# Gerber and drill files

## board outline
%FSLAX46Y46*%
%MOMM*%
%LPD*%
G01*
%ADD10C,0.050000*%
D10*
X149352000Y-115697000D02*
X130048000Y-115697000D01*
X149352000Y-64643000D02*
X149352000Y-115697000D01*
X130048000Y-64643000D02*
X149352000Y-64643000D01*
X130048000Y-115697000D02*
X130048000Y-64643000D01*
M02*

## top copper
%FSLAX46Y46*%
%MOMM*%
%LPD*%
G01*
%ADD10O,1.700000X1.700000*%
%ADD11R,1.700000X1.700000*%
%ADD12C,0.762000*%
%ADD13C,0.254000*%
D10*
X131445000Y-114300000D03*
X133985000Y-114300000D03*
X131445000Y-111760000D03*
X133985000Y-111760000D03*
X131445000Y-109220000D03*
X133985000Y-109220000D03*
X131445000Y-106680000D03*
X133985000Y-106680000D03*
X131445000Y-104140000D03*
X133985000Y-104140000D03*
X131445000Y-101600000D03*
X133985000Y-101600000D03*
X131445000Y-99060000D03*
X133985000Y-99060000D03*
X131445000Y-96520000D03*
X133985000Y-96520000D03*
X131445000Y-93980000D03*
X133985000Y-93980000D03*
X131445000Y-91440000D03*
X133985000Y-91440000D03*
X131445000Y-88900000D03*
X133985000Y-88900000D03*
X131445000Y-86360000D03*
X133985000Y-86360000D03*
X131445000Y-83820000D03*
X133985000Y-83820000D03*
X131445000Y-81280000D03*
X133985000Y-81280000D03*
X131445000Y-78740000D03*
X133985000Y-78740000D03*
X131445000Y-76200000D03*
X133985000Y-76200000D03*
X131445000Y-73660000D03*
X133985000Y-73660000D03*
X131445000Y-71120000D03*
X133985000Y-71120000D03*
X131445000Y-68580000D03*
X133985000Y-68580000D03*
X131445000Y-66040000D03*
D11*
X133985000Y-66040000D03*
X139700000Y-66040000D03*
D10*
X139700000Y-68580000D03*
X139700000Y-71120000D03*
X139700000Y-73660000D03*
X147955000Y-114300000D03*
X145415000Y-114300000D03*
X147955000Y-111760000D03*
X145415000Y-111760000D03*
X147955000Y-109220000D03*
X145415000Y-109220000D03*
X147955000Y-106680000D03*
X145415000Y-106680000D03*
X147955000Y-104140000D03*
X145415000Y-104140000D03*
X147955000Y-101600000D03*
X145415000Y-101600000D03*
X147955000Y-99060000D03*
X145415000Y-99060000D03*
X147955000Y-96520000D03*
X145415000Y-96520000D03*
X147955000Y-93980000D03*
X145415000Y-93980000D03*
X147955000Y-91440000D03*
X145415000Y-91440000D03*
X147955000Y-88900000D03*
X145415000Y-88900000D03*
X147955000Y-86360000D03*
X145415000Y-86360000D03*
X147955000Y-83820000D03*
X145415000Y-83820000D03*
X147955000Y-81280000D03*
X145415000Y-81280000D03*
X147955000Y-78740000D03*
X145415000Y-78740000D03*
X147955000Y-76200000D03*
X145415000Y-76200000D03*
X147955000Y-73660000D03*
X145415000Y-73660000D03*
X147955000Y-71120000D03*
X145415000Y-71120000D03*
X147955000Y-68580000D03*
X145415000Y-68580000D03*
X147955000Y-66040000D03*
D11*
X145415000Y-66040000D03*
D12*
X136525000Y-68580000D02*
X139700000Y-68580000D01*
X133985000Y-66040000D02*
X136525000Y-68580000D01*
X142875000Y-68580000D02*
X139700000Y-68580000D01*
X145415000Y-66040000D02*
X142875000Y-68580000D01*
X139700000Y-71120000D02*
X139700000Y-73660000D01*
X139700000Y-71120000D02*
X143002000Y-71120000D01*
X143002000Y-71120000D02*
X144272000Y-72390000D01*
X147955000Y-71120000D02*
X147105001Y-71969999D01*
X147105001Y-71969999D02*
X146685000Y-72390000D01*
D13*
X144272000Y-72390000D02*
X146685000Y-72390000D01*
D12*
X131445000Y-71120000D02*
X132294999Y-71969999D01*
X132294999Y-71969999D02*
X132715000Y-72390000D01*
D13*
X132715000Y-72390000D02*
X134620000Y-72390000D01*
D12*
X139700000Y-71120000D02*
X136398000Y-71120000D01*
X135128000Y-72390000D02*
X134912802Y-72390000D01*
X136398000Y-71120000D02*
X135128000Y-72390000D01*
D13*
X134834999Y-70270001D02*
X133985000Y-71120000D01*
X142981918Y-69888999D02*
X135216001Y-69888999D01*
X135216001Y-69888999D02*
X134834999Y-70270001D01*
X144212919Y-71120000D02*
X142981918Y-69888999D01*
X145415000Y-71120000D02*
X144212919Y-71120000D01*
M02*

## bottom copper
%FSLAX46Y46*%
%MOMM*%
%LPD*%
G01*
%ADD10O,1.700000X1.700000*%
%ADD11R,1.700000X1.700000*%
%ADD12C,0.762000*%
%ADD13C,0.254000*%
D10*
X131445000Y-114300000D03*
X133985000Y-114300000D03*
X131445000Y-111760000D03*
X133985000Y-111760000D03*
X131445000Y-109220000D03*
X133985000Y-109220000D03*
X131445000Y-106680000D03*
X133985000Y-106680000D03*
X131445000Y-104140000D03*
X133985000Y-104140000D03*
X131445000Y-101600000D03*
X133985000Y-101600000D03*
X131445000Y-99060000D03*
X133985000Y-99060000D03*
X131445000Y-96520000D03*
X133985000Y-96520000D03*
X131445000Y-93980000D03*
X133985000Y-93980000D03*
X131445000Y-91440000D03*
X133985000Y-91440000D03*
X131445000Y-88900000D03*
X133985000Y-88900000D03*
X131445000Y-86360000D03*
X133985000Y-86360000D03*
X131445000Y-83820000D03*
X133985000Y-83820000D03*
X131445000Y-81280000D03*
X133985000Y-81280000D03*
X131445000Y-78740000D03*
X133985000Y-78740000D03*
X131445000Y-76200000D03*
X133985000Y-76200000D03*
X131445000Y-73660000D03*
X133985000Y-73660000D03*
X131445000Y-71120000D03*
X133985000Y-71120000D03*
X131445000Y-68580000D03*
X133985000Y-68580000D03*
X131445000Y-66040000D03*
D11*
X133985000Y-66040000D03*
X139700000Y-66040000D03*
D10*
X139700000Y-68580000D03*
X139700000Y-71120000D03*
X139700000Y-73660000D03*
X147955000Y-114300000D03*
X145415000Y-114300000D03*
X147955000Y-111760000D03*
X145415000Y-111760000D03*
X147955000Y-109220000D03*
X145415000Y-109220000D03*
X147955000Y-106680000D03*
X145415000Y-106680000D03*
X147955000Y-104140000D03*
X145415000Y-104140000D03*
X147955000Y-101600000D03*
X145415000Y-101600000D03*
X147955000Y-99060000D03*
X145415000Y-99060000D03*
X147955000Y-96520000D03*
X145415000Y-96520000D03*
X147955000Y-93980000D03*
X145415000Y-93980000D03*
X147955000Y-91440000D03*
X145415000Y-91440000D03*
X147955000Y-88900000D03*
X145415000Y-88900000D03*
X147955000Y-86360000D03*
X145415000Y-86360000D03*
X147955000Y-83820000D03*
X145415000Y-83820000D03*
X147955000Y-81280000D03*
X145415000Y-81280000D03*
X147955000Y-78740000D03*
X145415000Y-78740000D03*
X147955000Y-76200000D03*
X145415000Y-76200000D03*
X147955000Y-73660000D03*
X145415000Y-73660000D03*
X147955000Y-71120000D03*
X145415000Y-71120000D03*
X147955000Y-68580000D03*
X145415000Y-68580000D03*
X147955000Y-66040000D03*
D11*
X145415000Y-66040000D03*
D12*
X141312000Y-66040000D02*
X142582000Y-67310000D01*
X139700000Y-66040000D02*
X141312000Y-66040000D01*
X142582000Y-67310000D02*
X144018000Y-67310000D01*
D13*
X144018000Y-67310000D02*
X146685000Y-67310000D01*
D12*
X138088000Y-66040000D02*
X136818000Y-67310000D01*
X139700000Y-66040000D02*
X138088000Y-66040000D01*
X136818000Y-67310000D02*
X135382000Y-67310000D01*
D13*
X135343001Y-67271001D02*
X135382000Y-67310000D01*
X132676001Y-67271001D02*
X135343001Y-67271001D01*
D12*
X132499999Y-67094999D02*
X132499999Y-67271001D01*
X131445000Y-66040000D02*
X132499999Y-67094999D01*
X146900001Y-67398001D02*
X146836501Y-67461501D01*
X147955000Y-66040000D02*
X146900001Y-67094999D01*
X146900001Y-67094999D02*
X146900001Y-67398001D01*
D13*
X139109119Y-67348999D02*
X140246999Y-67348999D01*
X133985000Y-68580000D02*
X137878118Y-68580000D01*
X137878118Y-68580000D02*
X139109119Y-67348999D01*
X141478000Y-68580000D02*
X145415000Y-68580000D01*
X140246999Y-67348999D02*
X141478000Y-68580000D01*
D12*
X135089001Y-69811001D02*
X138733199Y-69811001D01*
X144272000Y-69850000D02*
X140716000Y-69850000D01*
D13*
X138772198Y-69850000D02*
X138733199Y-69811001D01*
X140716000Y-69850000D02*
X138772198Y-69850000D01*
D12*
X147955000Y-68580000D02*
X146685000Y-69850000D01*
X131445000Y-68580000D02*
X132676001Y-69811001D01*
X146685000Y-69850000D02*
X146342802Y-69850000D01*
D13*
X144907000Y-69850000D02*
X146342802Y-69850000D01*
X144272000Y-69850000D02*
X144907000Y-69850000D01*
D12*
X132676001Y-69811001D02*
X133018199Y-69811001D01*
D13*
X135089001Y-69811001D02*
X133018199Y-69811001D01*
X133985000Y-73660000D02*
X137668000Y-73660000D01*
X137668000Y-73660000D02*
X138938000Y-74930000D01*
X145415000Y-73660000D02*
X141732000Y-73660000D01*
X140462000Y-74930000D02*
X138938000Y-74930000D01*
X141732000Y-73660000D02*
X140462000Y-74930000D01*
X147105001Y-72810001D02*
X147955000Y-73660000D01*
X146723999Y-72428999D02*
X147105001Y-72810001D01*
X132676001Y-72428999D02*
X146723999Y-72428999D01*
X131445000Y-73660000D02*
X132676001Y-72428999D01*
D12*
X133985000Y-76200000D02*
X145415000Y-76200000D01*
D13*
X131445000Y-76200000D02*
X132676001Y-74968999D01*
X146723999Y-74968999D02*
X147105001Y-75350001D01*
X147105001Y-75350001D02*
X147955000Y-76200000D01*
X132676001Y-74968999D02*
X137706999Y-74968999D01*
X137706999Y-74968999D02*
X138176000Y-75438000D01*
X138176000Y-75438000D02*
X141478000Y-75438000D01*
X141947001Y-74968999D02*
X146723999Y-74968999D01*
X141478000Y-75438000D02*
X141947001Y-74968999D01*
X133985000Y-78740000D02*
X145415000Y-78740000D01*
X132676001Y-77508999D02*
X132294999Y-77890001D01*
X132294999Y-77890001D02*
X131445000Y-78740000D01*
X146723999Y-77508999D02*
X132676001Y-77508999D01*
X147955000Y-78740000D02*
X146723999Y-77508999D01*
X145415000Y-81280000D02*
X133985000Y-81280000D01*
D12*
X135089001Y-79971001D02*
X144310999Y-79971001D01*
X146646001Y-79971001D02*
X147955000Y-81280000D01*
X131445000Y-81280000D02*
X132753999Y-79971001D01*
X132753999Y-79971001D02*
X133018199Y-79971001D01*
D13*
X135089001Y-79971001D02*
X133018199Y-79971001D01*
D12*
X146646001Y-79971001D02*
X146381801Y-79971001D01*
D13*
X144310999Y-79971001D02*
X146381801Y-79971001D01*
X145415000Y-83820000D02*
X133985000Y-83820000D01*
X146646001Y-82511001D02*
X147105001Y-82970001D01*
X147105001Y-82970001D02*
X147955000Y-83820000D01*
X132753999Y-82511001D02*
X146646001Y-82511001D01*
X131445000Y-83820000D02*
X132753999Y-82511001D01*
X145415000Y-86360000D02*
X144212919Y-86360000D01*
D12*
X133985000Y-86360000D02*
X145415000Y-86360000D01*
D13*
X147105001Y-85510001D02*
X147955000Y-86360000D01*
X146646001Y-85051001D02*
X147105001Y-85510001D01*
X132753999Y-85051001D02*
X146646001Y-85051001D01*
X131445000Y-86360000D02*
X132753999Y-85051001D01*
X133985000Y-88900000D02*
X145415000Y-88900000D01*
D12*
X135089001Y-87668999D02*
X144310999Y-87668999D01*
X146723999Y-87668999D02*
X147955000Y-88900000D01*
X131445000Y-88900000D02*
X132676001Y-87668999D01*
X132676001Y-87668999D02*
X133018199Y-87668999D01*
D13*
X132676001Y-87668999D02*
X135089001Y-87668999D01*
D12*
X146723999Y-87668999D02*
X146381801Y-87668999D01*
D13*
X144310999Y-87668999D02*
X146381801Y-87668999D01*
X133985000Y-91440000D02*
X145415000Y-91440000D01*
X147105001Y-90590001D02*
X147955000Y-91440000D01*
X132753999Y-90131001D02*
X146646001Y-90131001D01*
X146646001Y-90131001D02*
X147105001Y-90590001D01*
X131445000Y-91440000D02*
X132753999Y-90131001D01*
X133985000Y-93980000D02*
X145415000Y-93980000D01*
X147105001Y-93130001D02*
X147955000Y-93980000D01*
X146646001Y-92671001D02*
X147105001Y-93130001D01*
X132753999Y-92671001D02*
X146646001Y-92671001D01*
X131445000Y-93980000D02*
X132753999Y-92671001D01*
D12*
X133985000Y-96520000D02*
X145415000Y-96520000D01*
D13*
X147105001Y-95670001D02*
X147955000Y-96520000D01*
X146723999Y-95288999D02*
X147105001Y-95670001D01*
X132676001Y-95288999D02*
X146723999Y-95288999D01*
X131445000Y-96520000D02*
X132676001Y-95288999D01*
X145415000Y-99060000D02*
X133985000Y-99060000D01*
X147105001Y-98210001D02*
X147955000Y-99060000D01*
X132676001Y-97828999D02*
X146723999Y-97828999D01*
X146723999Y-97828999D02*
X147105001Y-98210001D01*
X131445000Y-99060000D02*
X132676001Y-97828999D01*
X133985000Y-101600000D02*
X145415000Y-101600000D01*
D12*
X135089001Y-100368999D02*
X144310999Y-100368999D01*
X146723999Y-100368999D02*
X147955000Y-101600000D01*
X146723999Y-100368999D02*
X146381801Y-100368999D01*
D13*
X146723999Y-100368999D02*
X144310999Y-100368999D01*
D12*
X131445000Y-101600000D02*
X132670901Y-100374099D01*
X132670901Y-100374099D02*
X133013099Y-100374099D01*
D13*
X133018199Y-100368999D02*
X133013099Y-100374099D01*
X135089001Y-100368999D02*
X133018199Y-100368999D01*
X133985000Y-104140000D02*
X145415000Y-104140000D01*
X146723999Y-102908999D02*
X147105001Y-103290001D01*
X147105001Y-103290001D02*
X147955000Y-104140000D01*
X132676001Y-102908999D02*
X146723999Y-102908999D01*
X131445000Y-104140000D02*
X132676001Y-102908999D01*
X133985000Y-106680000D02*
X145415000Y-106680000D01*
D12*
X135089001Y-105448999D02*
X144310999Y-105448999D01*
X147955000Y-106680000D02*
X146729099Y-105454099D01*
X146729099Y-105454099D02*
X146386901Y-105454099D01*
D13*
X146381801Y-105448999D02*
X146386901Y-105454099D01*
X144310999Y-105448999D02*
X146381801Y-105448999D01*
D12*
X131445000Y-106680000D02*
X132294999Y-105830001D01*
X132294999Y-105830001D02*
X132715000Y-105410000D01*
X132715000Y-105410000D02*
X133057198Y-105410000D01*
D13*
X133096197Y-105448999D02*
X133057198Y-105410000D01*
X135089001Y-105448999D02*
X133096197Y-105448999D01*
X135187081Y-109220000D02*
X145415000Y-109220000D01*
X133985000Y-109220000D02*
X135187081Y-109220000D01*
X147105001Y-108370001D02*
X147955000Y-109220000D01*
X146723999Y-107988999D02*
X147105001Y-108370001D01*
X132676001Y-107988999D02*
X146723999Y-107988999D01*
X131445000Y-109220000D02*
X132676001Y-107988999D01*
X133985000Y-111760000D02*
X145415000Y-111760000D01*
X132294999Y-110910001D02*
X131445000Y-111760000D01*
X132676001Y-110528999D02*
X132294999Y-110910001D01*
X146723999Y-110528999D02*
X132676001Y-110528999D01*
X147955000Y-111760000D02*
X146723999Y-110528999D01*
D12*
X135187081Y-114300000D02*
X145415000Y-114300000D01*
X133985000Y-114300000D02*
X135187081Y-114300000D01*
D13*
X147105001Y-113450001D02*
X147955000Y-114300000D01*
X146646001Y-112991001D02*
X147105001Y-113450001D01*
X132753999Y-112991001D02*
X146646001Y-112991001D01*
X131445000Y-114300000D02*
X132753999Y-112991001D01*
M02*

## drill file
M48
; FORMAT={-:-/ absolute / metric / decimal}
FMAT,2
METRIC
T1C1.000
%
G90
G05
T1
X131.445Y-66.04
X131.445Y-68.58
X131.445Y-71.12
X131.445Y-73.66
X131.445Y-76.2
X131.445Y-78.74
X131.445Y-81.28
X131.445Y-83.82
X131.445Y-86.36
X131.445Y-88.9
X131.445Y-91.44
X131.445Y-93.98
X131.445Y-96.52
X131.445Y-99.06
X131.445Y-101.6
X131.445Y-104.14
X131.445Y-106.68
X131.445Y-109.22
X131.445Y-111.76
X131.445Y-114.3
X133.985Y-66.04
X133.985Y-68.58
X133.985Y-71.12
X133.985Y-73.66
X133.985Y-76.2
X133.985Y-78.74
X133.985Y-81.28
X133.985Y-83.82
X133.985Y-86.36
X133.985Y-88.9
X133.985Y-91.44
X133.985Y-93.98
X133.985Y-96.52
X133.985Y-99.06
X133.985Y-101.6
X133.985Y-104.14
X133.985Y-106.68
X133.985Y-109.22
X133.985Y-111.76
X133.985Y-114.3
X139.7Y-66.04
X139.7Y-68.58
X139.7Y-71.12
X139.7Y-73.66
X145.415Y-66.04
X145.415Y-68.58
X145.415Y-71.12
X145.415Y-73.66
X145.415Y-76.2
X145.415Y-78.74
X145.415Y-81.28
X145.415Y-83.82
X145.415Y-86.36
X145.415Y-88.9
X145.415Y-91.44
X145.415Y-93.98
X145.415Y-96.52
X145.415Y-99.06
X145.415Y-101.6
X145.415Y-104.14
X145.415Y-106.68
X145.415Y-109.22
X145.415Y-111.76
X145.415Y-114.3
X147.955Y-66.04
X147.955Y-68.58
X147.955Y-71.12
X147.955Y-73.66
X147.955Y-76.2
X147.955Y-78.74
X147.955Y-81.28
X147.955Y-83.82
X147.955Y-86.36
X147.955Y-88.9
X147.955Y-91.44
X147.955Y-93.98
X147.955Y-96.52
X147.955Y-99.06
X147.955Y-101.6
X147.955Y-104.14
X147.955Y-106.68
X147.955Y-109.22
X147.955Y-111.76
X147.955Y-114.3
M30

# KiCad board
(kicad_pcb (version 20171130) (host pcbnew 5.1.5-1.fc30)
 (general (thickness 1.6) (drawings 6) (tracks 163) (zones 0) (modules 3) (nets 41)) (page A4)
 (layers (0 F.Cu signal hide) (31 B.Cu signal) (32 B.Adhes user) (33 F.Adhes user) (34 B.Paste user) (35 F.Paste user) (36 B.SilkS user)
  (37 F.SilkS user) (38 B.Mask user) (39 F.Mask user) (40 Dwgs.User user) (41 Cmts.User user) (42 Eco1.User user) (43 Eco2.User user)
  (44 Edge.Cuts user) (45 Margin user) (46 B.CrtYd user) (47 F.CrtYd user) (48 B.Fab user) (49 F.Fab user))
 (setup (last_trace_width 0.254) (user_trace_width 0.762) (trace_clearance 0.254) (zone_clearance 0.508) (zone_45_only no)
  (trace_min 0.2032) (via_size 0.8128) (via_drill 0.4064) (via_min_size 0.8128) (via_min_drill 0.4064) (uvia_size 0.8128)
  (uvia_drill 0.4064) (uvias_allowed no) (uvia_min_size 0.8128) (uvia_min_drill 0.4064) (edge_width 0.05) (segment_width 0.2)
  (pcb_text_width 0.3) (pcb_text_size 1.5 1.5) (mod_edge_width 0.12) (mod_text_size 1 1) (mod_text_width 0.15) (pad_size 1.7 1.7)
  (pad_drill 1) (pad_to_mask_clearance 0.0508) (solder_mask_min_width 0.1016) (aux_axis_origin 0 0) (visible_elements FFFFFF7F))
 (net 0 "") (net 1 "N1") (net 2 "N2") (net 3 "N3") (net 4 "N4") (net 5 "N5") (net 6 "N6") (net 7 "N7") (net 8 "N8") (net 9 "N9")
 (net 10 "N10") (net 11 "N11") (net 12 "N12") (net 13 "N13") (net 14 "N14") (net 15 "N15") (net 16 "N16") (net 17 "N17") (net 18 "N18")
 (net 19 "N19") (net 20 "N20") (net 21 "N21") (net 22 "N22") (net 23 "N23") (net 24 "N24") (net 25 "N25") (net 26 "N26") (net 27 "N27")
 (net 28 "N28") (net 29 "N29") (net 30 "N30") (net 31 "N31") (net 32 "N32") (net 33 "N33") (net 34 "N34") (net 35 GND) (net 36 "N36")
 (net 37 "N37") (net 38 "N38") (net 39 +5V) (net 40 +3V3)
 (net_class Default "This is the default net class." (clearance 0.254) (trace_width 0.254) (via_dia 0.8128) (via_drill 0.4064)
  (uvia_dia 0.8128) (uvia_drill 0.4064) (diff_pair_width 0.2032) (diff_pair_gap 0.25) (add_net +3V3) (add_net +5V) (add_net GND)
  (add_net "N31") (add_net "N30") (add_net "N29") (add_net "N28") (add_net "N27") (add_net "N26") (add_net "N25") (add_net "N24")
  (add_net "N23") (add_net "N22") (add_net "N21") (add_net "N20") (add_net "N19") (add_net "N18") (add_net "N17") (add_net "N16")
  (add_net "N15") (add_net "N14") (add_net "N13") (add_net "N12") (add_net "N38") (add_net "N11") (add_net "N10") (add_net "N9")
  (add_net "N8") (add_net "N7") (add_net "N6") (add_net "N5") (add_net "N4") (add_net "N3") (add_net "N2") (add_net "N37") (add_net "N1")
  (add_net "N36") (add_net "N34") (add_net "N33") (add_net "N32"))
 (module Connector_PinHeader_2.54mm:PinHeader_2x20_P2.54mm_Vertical (layer B.Cu) (at 133.985 66.04 180)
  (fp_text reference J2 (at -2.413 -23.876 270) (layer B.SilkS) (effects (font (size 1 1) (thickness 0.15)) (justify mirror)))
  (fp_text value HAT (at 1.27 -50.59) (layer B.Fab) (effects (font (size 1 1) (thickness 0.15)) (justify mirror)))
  (pad 40 thru_hole oval (at 2.54 -48.26 180) (size 1.7 1.7) (drill 1) (layers *.Cu *.Mask) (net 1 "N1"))
  (pad 39 thru_hole oval (at 0 -48.26 180) (size 1.7 1.7) (drill 1) (layers *.Cu *.Mask) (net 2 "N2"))
  (pad 38 thru_hole oval (at 2.54 -45.72 180) (size 1.7 1.7) (drill 1) (layers *.Cu *.Mask) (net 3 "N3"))
  (pad 37 thru_hole oval (at 0 -45.72 180) (size 1.7 1.7) (drill 1) (layers *.Cu *.Mask) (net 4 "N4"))
  (pad 36 thru_hole oval (at 2.54 -43.18 180) (size 1.7 1.7) (drill 1) (layers *.Cu *.Mask) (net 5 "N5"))
  (pad 35 thru_hole oval (at 0 -43.18 180) (size 1.7 1.7) (drill 1) (layers *.Cu *.Mask) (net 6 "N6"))
  (pad 34 thru_hole oval (at 2.54 -40.64 180) (size 1.7 1.7) (drill 1) (layers *.Cu *.Mask) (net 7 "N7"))
  (pad 33 thru_hole oval (at 0 -40.64 180) (size 1.7 1.7) (drill 1) (layers *.Cu *.Mask) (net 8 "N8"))
  (pad 32 thru_hole oval (at 2.54 -38.1 180) (size 1.7 1.7) (drill 1) (layers *.Cu *.Mask) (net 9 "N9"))
  (pad 31 thru_hole oval (at 0 -38.1 180) (size 1.7 1.7) (drill 1) (layers *.Cu *.Mask) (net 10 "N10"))
  (pad 30 thru_hole oval (at 2.54 -35.56 180) (size 1.7 1.7) (drill 1) (layers *.Cu *.Mask) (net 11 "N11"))
  (pad 29 thru_hole oval (at 0 -35.56 180) (size 1.7 1.7) (drill 1) (layers *.Cu *.Mask) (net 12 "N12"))
  (pad 28 thru_hole oval (at 2.54 -33.02 180) (size 1.7 1.7) (drill 1) (layers *.Cu *.Mask) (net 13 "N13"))
  (pad 27 thru_hole oval (at 0 -33.02 180) (size 1.7 1.7) (drill 1) (layers *.Cu *.Mask) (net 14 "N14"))
  (pad 26 thru_hole oval (at 2.54 -30.48 180) (size 1.7 1.7) (drill 1) (layers *.Cu *.Mask) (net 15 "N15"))
  (pad 25 thru_hole oval (at 0 -30.48 180) (size 1.7 1.7) (drill 1) (layers *.Cu *.Mask) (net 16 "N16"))
  (pad 24 thru_hole oval (at 2.54 -27.94 180) (size 1.7 1.7) (drill 1) (layers *.Cu *.Mask) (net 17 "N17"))
  (pad 23 thru_hole oval (at 0 -27.94 180) (size 1.7 1.7) (drill 1) (layers *.Cu *.Mask) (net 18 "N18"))
  (pad 22 thru_hole oval (at 2.54 -25.4 180) (size 1.7 1.7) (drill 1) (layers *.Cu *.Mask) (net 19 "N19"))
  (pad 21 thru_hole oval (at 0 -25.4 180) (size 1.7 1.7) (drill 1) (layers *.Cu *.Mask) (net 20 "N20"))
  (pad 20 thru_hole oval (at 2.54 -22.86 180) (size 1.7 1.7) (drill 1) (layers *.Cu *.Mask) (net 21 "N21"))
  (pad 19 thru_hole oval (at 0 -22.86 180) (size 1.7 1.7) (drill 1) (layers *.Cu *.Mask) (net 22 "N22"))
  (pad 18 thru_hole oval (at 2.54 -20.32 180) (size 1.7 1.7) (drill 1) (layers *.Cu *.Mask) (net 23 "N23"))
  (pad 17 thru_hole oval (at 0 -20.32 180) (size 1.7 1.7) (drill 1) (layers *.Cu *.Mask) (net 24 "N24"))
  (pad 16 thru_hole oval (at 2.54 -17.78 180) (size 1.7 1.7) (drill 1) (layers *.Cu *.Mask) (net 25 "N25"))
  (pad 15 thru_hole oval (at 0 -17.78 180) (size 1.7 1.7) (drill 1) (layers *.Cu *.Mask) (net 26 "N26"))
  (pad 14 thru_hole oval (at 2.54 -15.24 180) (size 1.7 1.7) (drill 1) (layers *.Cu *.Mask) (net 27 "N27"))
  (pad 13 thru_hole oval (at 0 -15.24 180) (size 1.7 1.7) (drill 1) (layers *.Cu *.Mask) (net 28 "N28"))
  (pad 12 thru_hole oval (at 2.54 -12.7 180) (size 1.7 1.7) (drill 1) (layers *.Cu *.Mask) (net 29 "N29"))
  (pad 11 thru_hole oval (at 0 -12.7 180) (size 1.7 1.7) (drill 1) (layers *.Cu *.Mask) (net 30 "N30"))
  (pad 10 thru_hole oval (at 2.54 -10.16 180) (size 1.7 1.7) (drill 1) (layers *.Cu *.Mask) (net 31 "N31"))
  (pad 9 thru_hole oval (at 0 -10.16 180) (size 1.7 1.7) (drill 1) (layers *.Cu *.Mask) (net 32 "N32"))
  (pad 8 thru_hole oval (at 2.54 -7.62 180) (size 1.7 1.7) (drill 1) (layers *.Cu *.Mask) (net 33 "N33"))
  (pad 7 thru_hole oval (at 0 -7.62 180) (size 1.7 1.7) (drill 1) (layers *.Cu *.Mask) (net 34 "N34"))
  (pad 6 thru_hole oval (at 2.54 -5.08 180) (size 1.7 1.7) (drill 1) (layers *.Cu *.Mask) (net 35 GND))
  (pad 5 thru_hole oval (at 0 -5.08 180) (size 1.7 1.7) (drill 1) (layers *.Cu *.Mask) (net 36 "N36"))
  (pad 4 thru_hole oval (at 2.54 -2.54 180) (size 1.7 1.7) (drill 1) (layers *.Cu *.Mask) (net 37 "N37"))
  (pad 3 thru_hole oval (at 0 -2.54 180) (size 1.7 1.7) (drill 1) (layers *.Cu *.Mask) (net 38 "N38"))
  (pad 2 thru_hole oval (at 2.54 0 180) (size 1.7 1.7) (drill 1) (layers *.Cu *.Mask) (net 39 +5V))
  (pad 1 thru_hole rect (at 0 0 180) (size 1.7 1.7) (drill 1) (layers *.Cu *.Mask) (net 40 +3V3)))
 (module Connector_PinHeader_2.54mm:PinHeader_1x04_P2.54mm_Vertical (layer F.Cu) (at 139.7 66.04)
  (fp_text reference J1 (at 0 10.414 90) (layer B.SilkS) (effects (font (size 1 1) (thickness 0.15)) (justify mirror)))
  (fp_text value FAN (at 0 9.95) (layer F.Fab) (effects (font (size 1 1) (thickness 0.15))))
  (pad 1 thru_hole rect (at 0 0) (size 1.7 1.7) (drill 1) (layers *.Cu *.Mask) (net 39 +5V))
  (pad 2 thru_hole oval (at 0 2.54) (size 1.7 1.7) (drill 1) (layers *.Cu *.Mask) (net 40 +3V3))
  (pad 3 thru_hole oval (at 0 5.08) (size 1.7 1.7) (drill 1) (layers *.Cu *.Mask) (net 35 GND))
  (pad 4 thru_hole oval (at 0 7.62) (size 1.7 1.7) (drill 1) (layers *.Cu *.Mask) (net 35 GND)))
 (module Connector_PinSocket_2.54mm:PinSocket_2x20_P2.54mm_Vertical (layer B.Cu) (at 145.415 66.04 180)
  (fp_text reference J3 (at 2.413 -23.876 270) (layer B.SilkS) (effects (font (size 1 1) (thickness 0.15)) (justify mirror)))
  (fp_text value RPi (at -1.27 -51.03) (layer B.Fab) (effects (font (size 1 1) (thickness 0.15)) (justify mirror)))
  (pad 40 thru_hole oval (at -2.54 -48.26 180) (size 1.7 1.7) (drill 1) (layers *.Cu *.Mask) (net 1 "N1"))
  (pad 39 thru_hole oval (at 0 -48.26 180) (size 1.7 1.7) (drill 1) (layers *.Cu *.Mask) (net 2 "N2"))
  (pad 38 thru_hole oval (at -2.54 -45.72 180) (size 1.7 1.7) (drill 1) (layers *.Cu *.Mask) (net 3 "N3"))
  (pad 37 thru_hole oval (at 0 -45.72 180) (size 1.7 1.7) (drill 1) (layers *.Cu *.Mask) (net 4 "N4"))
  (pad 36 thru_hole oval (at -2.54 -43.18 180) (size 1.7 1.7) (drill 1) (layers *.Cu *.Mask) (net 5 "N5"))
  (pad 35 thru_hole oval (at 0 -43.18 180) (size 1.7 1.7) (drill 1) (layers *.Cu *.Mask) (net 6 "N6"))
  (pad 34 thru_hole oval (at -2.54 -40.64 180) (size 1.7 1.7) (drill 1) (layers *.Cu *.Mask) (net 7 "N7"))
  (pad 33 thru_hole oval (at 0 -40.64 180) (size 1.7 1.7) (drill 1) (layers *.Cu *.Mask) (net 8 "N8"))
  (pad 32 thru_hole oval (at -2.54 -38.1 180) (size 1.7 1.7) (drill 1) (layers *.Cu *.Mask) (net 9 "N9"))
  (pad 31 thru_hole oval (at 0 -38.1 180) (size 1.7 1.7) (drill 1) (layers *.Cu *.Mask) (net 10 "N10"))
  (pad 30 thru_hole oval (at -2.54 -35.56 180) (size 1.7 1.7) (drill 1) (layers *.Cu *.Mask) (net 11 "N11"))
  (pad 29 thru_hole oval (at 0 -35.56 180) (size 1.7 1.7) (drill 1) (layers *.Cu *.Mask) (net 12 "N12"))
  (pad 28 thru_hole oval (at -2.54 -33.02 180) (size 1.7 1.7) (drill 1) (layers *.Cu *.Mask) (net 13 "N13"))
  (pad 27 thru_hole oval (at 0 -33.02 180) (size 1.7 1.7) (drill 1) (layers *.Cu *.Mask) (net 14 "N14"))
  (pad 26 thru_hole oval (at -2.54 -30.48 180) (size 1.7 1.7) (drill 1) (layers *.Cu *.Mask) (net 15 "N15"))
  (pad 25 thru_hole oval (at 0 -30.48 180) (size 1.7 1.7) (drill 1) (layers *.Cu *.Mask) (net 16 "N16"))
  (pad 24 thru_hole oval (at -2.54 -27.94 180) (size 1.7 1.7) (drill 1) (layers *.Cu *.Mask) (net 17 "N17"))
  (pad 23 thru_hole oval (at 0 -27.94 180) (size 1.7 1.7) (drill 1) (layers *.Cu *.Mask) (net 18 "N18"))
  (pad 22 thru_hole oval (at -2.54 -25.4 180) (size 1.7 1.7) (drill 1) (layers *.Cu *.Mask) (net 19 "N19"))
  (pad 21 thru_hole oval (at 0 -25.4 180) (size 1.7 1.7) (drill 1) (layers *.Cu *.Mask) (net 20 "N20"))
  (pad 20 thru_hole oval (at -2.54 -22.86 180) (size 1.7 1.7) (drill 1) (layers *.Cu *.Mask) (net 21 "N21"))
  (pad 19 thru_hole oval (at 0 -22.86 180) (size 1.7 1.7) (drill 1) (layers *.Cu *.Mask) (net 22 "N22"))
  (pad 18 thru_hole oval (at -2.54 -20.32 180) (size 1.7 1.7) (drill 1) (layers *.Cu *.Mask) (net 23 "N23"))
  (pad 17 thru_hole oval (at 0 -20.32 180) (size 1.7 1.7) (drill 1) (layers *.Cu *.Mask) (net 24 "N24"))
  (pad 16 thru_hole oval (at -2.54 -17.78 180) (size 1.7 1.7) (drill 1) (layers *.Cu *.Mask) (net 25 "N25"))
  (pad 15 thru_hole oval (at 0 -17.78 180) (size 1.7 1.7) (drill 1) (layers *.Cu *.Mask) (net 26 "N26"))
  (pad 14 thru_hole oval (at -2.54 -15.24 180) (size 1.7 1.7) (drill 1) (layers *.Cu *.Mask) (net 27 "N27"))
  (pad 13 thru_hole oval (at 0 -15.24 180) (size 1.7 1.7) (drill 1) (layers *.Cu *.Mask) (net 28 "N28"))
  (pad 12 thru_hole oval (at -2.54 -12.7 180) (size 1.7 1.7) (drill 1) (layers *.Cu *.Mask) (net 29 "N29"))
  (pad 11 thru_hole oval (at 0 -12.7 180) (size 1.7 1.7) (drill 1) (layers *.Cu *.Mask) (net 30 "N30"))
  (pad 10 thru_hole oval (at -2.54 -10.16 180) (size 1.7 1.7) (drill 1) (layers *.Cu *.Mask) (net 31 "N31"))
  (pad 9 thru_hole oval (at 0 -10.16 180) (size 1.7 1.7) (drill 1) (layers *.Cu *.Mask) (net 32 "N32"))
  (pad 8 thru_hole oval (at -2.54 -7.62 180) (size 1.7 1.7) (drill 1) (layers *.Cu *.Mask) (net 33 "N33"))
  (pad 7 thru_hole oval (at 0 -7.62 180) (size 1.7 1.7) (drill 1) (layers *.Cu *.Mask) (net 34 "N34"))
  (pad 6 thru_hole oval (at -2.54 -5.08 180) (size 1.7 1.7) (drill 1) (layers *.Cu *.Mask) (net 35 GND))
  (pad 5 thru_hole oval (at 0 -5.08 180) (size 1.7 1.7) (drill 1) (layers *.Cu *.Mask) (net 36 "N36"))
  (pad 4 thru_hole oval (at -2.54 -2.54 180) (size 1.7 1.7) (drill 1) (layers *.Cu *.Mask) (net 37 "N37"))
  (pad 3 thru_hole oval (at 0 -2.54 180) (size 1.7 1.7) (drill 1) (layers *.Cu *.Mask) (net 38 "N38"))
  (pad 2 thru_hole oval (at -2.54 0 180) (size 1.7 1.7) (drill 1) (layers *.Cu *.Mask) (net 39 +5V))
  (pad 1 thru_hole rect (at 0 0 180) (size 1.7 1.7) (drill 1) (layers *.Cu *.Mask) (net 40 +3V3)))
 (gr_line (start 149.352 115.697) (end 130.048 115.697) (layer Edge.Cuts) (width 0.05))
 (gr_line (start 149.352 64.643) (end 149.352 115.697) (layer Edge.Cuts) (width 0.05))
 (gr_line (start 130.048 64.643) (end 149.352 64.643) (layer Edge.Cuts) (width 0.05))
 (gr_line (start 130.048 115.697) (end 130.048 64.643) (layer Edge.Cuts) (width 0.05))
 (segment (start 136.525 68.58) (end 139.7 68.58) (width 0.762) (layer F.Cu) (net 40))
 (segment (start 133.985 66.04) (end 136.525 68.58) (width 0.762) (layer F.Cu) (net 40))
 (segment (start 142.875 68.58) (end 139.7 68.58) (width 0.762) (layer F.Cu) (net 40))
 (segment (start 145.415 66.04) (end 142.875 68.58) (width 0.762) (layer F.Cu) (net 40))
 (segment (start 141.312 66.04) (end 142.582 67.31) (width 0.762) (layer B.Cu) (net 39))
 (segment (start 139.7 66.04) (end 141.312 66.04) (width 0.762) (layer B.Cu) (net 39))
 (segment (start 142.582 67.31) (end 144.018 67.31) (width 0.762) (layer B.Cu) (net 39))
 (segment (start 144.018 67.31) (end 146.685 67.31) (width 0.254) (layer B.Cu) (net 39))
 (segment (start 138.088 66.04) (end 136.818 67.31) (width 0.762) (layer B.Cu) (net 39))
 (segment (start 139.7 66.04) (end 138.088 66.04) (width 0.762) (layer B.Cu) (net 39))
 (segment (start 136.818 67.31) (end 135.382 67.31) (width 0.762) (layer B.Cu) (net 39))
 (segment (start 135.343001 67.271001) (end 135.382 67.31) (width 0.254) (layer B.Cu) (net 39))
 (segment (start 132.676001 67.271001) (end 135.343001 67.271001) (width 0.254) (layer B.Cu) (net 39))
 (segment (start 132.499999 67.094999) (end 132.499999 67.271001) (width 0.762) (layer B.Cu) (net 39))
 (segment (start 131.445 66.04) (end 132.499999 67.094999) (width 0.762) (layer B.Cu) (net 39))
 (segment (start 146.900001 67.398001) (end 146.836501 67.461501) (width 0.762) (layer B.Cu) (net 39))
 (segment (start 147.955 66.04) (end 146.900001 67.094999) (width 0.762) (layer B.Cu) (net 39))
 (segment (start 146.900001 67.094999) (end 146.900001 67.398001) (width 0.762) (layer B.Cu) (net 39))
 (segment (start 139.7 71.12) (end 139.7 73.66) (width 0.762) (layer F.Cu) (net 35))
 (segment (start 139.7 71.12) (end 143.002 71.12) (width 0.762) (layer F.Cu) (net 35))
 (segment (start 143.002 71.12) (end 144.272 72.39) (width 0.762) (layer F.Cu) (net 35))
 (segment (start 147.955 71.12) (end 147.105001 71.969999) (width 0.762) (layer F.Cu) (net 35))
 (segment (start 147.105001 71.969999) (end 146.685 72.39) (width 0.762) (layer F.Cu) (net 35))
 (segment (start 144.272 72.39) (end 146.685 72.39) (width 0.254) (layer F.Cu) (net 35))
 (segment (start 131.445 71.12) (end 132.294999 71.969999) (width 0.762) (layer F.Cu) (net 35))
 (segment (start 132.294999 71.969999) (end 132.715 72.39) (width 0.762) (layer F.Cu) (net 35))
 (segment (start 132.715 72.39) (end 134.62 72.39) (width 0.254) (layer F.Cu) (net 35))
 (segment (start 139.7 71.12) (end 136.398 71.12) (width 0.762) (layer F.Cu) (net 35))
 (segment (start 135.128 72.39) (end 134.912802 72.39) (width 0.762) (layer F.Cu) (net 35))
 (segment (start 136.398 71.12) (end 135.128 72.39) (width 0.762) (layer F.Cu) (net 35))
 (segment (start 139.109119 67.348999) (end 140.246999 67.348999) (width 0.254) (layer B.Cu) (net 38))
 (segment (start 133.985 68.58) (end 137.878118 68.58) (width 0.254) (layer B.Cu) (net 38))
 (segment (start 137.878118 68.58) (end 139.109119 67.348999) (width 0.254) (layer B.Cu) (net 38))
 (segment (start 141.478 68.58) (end 145.415 68.58) (width 0.254) (layer B.Cu) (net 38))
 (segment (start 140.246999 67.348999) (end 141.478 68.58) (width 0.254) (layer B.Cu) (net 38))
 (segment (start 135.089001 69.811001) (end 138.733199 69.811001) (width 0.762) (layer B.Cu) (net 37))
 (segment (start 144.272 69.85) (end 140.716 69.85) (width 0.762) (layer B.Cu) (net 37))
 (segment (start 138.772198 69.85) (end 138.733199 69.811001) (width 0.254) (layer B.Cu) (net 37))
 (segment (start 140.716 69.85) (end 138.772198 69.85) (width 0.254) (layer B.Cu) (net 37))
 (segment (start 147.955 68.58) (end 146.685 69.85) (width 0.762) (layer B.Cu) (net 37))
 (segment (start 131.445 68.58) (end 132.676001 69.811001) (width 0.762) (layer B.Cu) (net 37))
 (segment (start 146.685 69.85) (end 146.342802 69.85) (width 0.762) (layer B.Cu) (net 37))
 (segment (start 144.907 69.85) (end 146.342802 69.85) (width 0.254) (layer B.Cu) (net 37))
 (segment (start 144.272 69.85) (end 144.907 69.85) (width 0.254) (layer B.Cu) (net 37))
 (segment (start 132.676001 69.811001) (end 133.018199 69.811001) (width 0.762) (layer B.Cu) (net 37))
 (segment (start 135.089001 69.811001) (end 133.018199 69.811001) (width 0.254) (layer B.Cu) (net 37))
 (segment (start 133.985 73.66) (end 137.668 73.66) (width 0.254) (layer B.Cu) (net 34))
 (segment (start 137.668 73.66) (end 138.938 74.93) (width 0.254) (layer B.Cu) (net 34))
 (segment (start 145.415 73.66) (end 141.732 73.66) (width 0.254) (layer B.Cu) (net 34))
 (segment (start 140.462 74.93) (end 138.938 74.93) (width 0.254) (layer B.Cu) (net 34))
 (segment (start 141.732 73.66) (end 140.462 74.93) (width 0.254) (layer B.Cu) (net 34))
 (segment (start 147.105001 72.810001) (end 147.955 73.66) (width 0.254) (layer B.Cu) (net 33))
 (segment (start 146.723999 72.428999) (end 147.105001 72.810001) (width 0.254) (layer B.Cu) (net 33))
 (segment (start 132.676001 72.428999) (end 146.723999 72.428999) (width 0.254) (layer B.Cu) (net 33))
 (segment (start 131.445 73.66) (end 132.676001 72.428999) (width 0.254) (layer B.Cu) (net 33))
 (segment (start 133.985 76.2) (end 145.415 76.2) (width 0.762) (layer B.Cu) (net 32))
 (segment (start 131.445 76.2) (end 132.676001 74.968999) (width 0.254) (layer B.Cu) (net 31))
 (segment (start 146.723999 74.968999) (end 147.105001 75.350001) (width 0.254) (layer B.Cu) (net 31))
 (segment (start 147.105001 75.350001) (end 147.955 76.2) (width 0.254) (layer B.Cu) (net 31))
 (segment (start 132.676001 74.968999) (end 137.706999 74.968999) (width 0.254) (layer B.Cu) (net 31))
 (segment (start 137.706999 74.968999) (end 138.176 75.438) (width 0.254) (layer B.Cu) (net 31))
 (segment (start 138.176 75.438) (end 141.478 75.438) (width 0.254) (layer B.Cu) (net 31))
 (segment (start 141.947001 74.968999) (end 146.723999 74.968999) (width 0.254) (layer B.Cu) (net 31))
 (segment (start 141.478 75.438) (end 141.947001 74.968999) (width 0.254) (layer B.Cu) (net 31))
 (segment (start 133.985 78.74) (end 145.415 78.74) (width 0.254) (layer B.Cu) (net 30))
 (segment (start 132.676001 77.508999) (end 132.294999 77.890001) (width 0.254) (layer B.Cu) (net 29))
 (segment (start 132.294999 77.890001) (end 131.445 78.74) (width 0.254) (layer B.Cu) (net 29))
 (segment (start 146.723999 77.508999) (end 132.676001 77.508999) (width 0.254) (layer B.Cu) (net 29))
 (segment (start 147.955 78.74) (end 146.723999 77.508999) (width 0.254) (layer B.Cu) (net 29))
 (segment (start 145.415 81.28) (end 133.985 81.28) (width 0.254) (layer B.Cu) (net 28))
 (segment (start 135.089001 79.971001) (end 144.310999 79.971001) (width 0.762) (layer B.Cu) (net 27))
 (segment (start 146.646001 79.971001) (end 147.955 81.28) (width 0.762) (layer B.Cu) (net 27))
 (segment (start 131.445 81.28) (end 132.753999 79.971001) (width 0.762) (layer B.Cu) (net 27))
 (segment (start 132.753999 79.971001) (end 133.018199 79.971001) (width 0.762) (layer B.Cu) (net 27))
 (segment (start 135.089001 79.971001) (end 133.018199 79.971001) (width 0.254) (layer B.Cu) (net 27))
 (segment (start 146.646001 79.971001) (end 146.381801 79.971001) (width 0.762) (layer B.Cu) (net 27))
 (segment (start 144.310999 79.971001) (end 146.381801 79.971001) (width 0.254) (layer B.Cu) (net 27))
 (segment (start 145.415 83.82) (end 133.985 83.82) (width 0.254) (layer B.Cu) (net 26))
 (segment (start 146.646001 82.511001) (end 147.105001 82.970001) (width 0.254) (layer B.Cu) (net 25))
 (segment (start 147.105001 82.970001) (end 147.955 83.82) (width 0.254) (layer B.Cu) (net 25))
 (segment (start 132.753999 82.511001) (end 146.646001 82.511001) (width 0.254) (layer B.Cu) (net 25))
 (segment (start 131.445 83.82) (end 132.753999 82.511001) (width 0.254) (layer B.Cu) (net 25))
 (segment (start 145.415 86.36) (end 144.212919 86.36) (width 0.254) (layer B.Cu) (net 24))
 (segment (start 133.985 86.36) (end 145.415 86.36) (width 0.762) (layer B.Cu) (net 24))
 (segment (start 147.105001 85.510001) (end 147.955 86.36) (width 0.254) (layer B.Cu) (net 23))
 (segment (start 146.646001 85.051001) (end 147.105001 85.510001) (width 0.254) (layer B.Cu) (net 23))
 (segment (start 132.753999 85.051001) (end 146.646001 85.051001) (width 0.254) (layer B.Cu) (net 23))
 (segment (start 131.445 86.36) (end 132.753999 85.051001) (width 0.254) (layer B.Cu) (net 23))
 (segment (start 133.985 88.9) (end 145.415 88.9) (width 0.254) (layer B.Cu) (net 22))
 (segment (start 135.089001 87.668999) (end 144.310999 87.668999) (width 0.762) (layer B.Cu) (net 21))
 (segment (start 146.723999 87.668999) (end 147.955 88.9) (width 0.762) (layer B.Cu) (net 21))
 (segment (start 131.445 88.9) (end 132.676001 87.668999) (width 0.762) (layer B.Cu) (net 21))
 (segment (start 132.676001 87.668999) (end 133.018199 87.668999) (width 0.762) (layer B.Cu) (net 21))
 (segment (start 132.676001 87.668999) (end 135.089001 87.668999) (width 0.254) (layer B.Cu) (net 21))
 (segment (start 146.723999 87.668999) (end 146.381801 87.668999) (width 0.762) (layer B.Cu) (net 21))
 (segment (start 144.310999 87.668999) (end 146.381801 87.668999) (width 0.254) (layer B.Cu) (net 21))
 (segment (start 133.985 91.44) (end 145.415 91.44) (width 0.254) (layer B.Cu) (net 20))
 (segment (start 147.105001 90.590001) (end 147.955 91.44) (width 0.254) (layer B.Cu) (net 19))
 (segment (start 132.753999 90.131001) (end 146.646001 90.131001) (width 0.254) (layer B.Cu) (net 19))
 (segment (start 146.646001 90.131001) (end 147.105001 90.590001) (width 0.254) (layer B.Cu) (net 19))
 (segment (start 131.445 91.44) (end 132.753999 90.131001) (width 0.254) (layer B.Cu) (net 19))
 (segment (start 133.985 93.98) (end 145.415 93.98) (width 0.254) (layer B.Cu) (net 18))
 (segment (start 147.105001 93.130001) (end 147.955 93.98) (width 0.254) (layer B.Cu) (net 17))
 (segment (start 146.646001 92.671001) (end 147.105001 93.130001) (width 0.254) (layer B.Cu) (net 17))
 (segment (start 132.753999 92.671001) (end 146.646001 92.671001) (width 0.254) (layer B.Cu) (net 17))
 (segment (start 131.445 93.98) (end 132.753999 92.671001) (width 0.254) (layer B.Cu) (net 17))
 (segment (start 133.985 96.52) (end 145.415 96.52) (width 0.762) (layer B.Cu) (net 16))
 (segment (start 147.105001 95.670001) (end 147.955 96.52) (width 0.254) (layer B.Cu) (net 15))
 (segment (start 146.723999 95.288999) (end 147.105001 95.670001) (width 0.254) (layer B.Cu) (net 15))
 (segment (start 132.676001 95.288999) (end 146.723999 95.288999) (width 0.254) (layer B.Cu) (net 15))
 (segment (start 131.445 96.52) (end 132.676001 95.288999) (width 0.254) (layer B.Cu) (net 15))
 (segment (start 145.415 99.06) (end 133.985 99.06) (width 0.254) (layer B.Cu) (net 14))
 (segment (start 147.105001 98.210001) (end 147.955 99.06) (width 0.254) (layer B.Cu) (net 13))
 (segment (start 132.676001 97.828999) (end 146.723999 97.828999) (width 0.254) (layer B.Cu) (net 13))
 (segment (start 146.723999 97.828999) (end 147.105001 98.210001) (width 0.254) (layer B.Cu) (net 13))
 (segment (start 131.445 99.06) (end 132.676001 97.828999) (width 0.254) (layer B.Cu) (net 13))
 (segment (start 133.985 101.6) (end 145.415 101.6) (width 0.254) (layer B.Cu) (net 12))
 (segment (start 135.089001 100.368999) (end 144.310999 100.368999) (width 0.762) (layer B.Cu) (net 11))
 (segment (start 146.723999 100.368999) (end 147.955 101.6) (width 0.762) (layer B.Cu) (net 11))
 (segment (start 146.723999 100.368999) (end 146.381801 100.368999) (width 0.762) (layer B.Cu) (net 11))
 (segment (start 146.723999 100.368999) (end 144.310999 100.368999) (width 0.254) (layer B.Cu) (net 11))
 (segment (start 131.445 101.6) (end 132.670901 100.374099) (width 0.762) (layer B.Cu) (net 11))
 (segment (start 132.670901 100.374099) (end 133.013099 100.374099) (width 0.762) (layer B.Cu) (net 11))
 (segment (start 133.018199 100.368999) (end 133.013099 100.374099) (width 0.254) (layer B.Cu) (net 11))
 (segment (start 135.089001 100.368999) (end 133.018199 100.368999) (width 0.254) (layer B.Cu) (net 11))
 (segment (start 133.985 104.14) (end 145.415 104.14) (width 0.254) (layer B.Cu) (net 10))
 (segment (start 146.723999 102.908999) (end 147.105001 103.290001) (width 0.254) (layer B.Cu) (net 9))
 (segment (start 147.105001 103.290001) (end 147.955 104.14) (width 0.254) (layer B.Cu) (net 9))
 (segment (start 132.676001 102.908999) (end 146.723999 102.908999) (width 0.254) (layer B.Cu) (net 9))
 (segment (start 131.445 104.14) (end 132.676001 102.908999) (width 0.254) (layer B.Cu) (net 9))
 (segment (start 133.985 106.68) (end 145.415 106.68) (width 0.254) (layer B.Cu) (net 8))
 (segment (start 135.089001 105.448999) (end 144.310999 105.448999) (width 0.762) (layer B.Cu) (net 7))
 (segment (start 147.955 106.68) (end 146.729099 105.454099) (width 0.762) (layer B.Cu) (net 7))
 (segment (start 146.729099 105.454099) (end 146.386901 105.454099) (width 0.762) (layer B.Cu) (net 7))
 (segment (start 146.381801 105.448999) (end 146.386901 105.454099) (width 0.254) (layer B.Cu) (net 7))
 (segment (start 144.310999 105.448999) (end 146.381801 105.448999) (width 0.254) (layer B.Cu) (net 7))
 (segment (start 131.445 106.68) (end 132.294999 105.830001) (width 0.762) (layer B.Cu) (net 7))
 (segment (start 132.294999 105.830001) (end 132.715 105.41) (width 0.762) (layer B.Cu) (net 7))
 (segment (start 132.715 105.41) (end 133.057198 105.41) (width 0.762) (layer B.Cu) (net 7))
 (segment (start 133.096197 105.448999) (end 133.057198 105.41) (width 0.254) (layer B.Cu) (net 7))
 (segment (start 135.089001 105.448999) (end 133.096197 105.448999) (width 0.254) (layer B.Cu) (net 7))
 (segment (start 135.187081 109.22) (end 145.415 109.22) (width 0.254) (layer B.Cu) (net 6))
 (segment (start 133.985 109.22) (end 135.187081 109.22) (width 0.254) (layer B.Cu) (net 6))
 (segment (start 147.105001 108.370001) (end 147.955 109.22) (width 0.254) (layer B.Cu) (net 5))
 (segment (start 146.723999 107.988999) (end 147.105001 108.370001) (width 0.254) (layer B.Cu) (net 5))
 (segment (start 132.676001 107.988999) (end 146.723999 107.988999) (width 0.254) (layer B.Cu) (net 5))
 (segment (start 131.445 109.22) (end 132.676001 107.988999) (width 0.254) (layer B.Cu) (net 5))
 (segment (start 133.985 111.76) (end 145.415 111.76) (width 0.254) (layer B.Cu) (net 4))
 (segment (start 132.294999 110.910001) (end 131.445 111.76) (width 0.254) (layer B.Cu) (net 3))
 (segment (start 132.676001 110.528999) (end 132.294999 110.910001) (width 0.254) (layer B.Cu) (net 3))
 (segment (start 146.723999 110.528999) (end 132.676001 110.528999) (width 0.254) (layer B.Cu) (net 3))
 (segment (start 147.955 111.76) (end 146.723999 110.528999) (width 0.254) (layer B.Cu) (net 3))
 (segment (start 135.187081 114.3) (end 145.415 114.3) (width 0.762) (layer B.Cu) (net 2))
 (segment (start 133.985 114.3) (end 135.187081 114.3) (width 0.762) (layer B.Cu) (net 2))
 (segment (start 147.105001 113.450001) (end 147.955 114.3) (width 0.254) (layer B.Cu) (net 1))
 (segment (start 146.646001 112.991001) (end 147.105001 113.450001) (width 0.254) (layer B.Cu) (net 1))
 (segment (start 132.753999 112.991001) (end 146.646001 112.991001) (width 0.254) (layer B.Cu) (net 1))
 (segment (start 131.445 114.3) (end 132.753999 112.991001) (width 0.254) (layer B.Cu) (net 1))
 (segment (start 134.834999 70.270001) (end 133.985 71.12) (width 0.254) (layer F.Cu) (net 36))
 (segment (start 142.981918 69.888999) (end 135.216001 69.888999) (width 0.254) (layer F.Cu) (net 36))
 (segment (start 135.216001 69.888999) (end 134.834999 70.270001) (width 0.254) (layer F.Cu) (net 36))
 (segment (start 144.212919 71.12) (end 142.981918 69.888999) (width 0.254) (layer F.Cu) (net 36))
 (segment (start 145.415 71.12) (end 144.212919 71.12) (width 0.254) (layer F.Cu) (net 36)))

